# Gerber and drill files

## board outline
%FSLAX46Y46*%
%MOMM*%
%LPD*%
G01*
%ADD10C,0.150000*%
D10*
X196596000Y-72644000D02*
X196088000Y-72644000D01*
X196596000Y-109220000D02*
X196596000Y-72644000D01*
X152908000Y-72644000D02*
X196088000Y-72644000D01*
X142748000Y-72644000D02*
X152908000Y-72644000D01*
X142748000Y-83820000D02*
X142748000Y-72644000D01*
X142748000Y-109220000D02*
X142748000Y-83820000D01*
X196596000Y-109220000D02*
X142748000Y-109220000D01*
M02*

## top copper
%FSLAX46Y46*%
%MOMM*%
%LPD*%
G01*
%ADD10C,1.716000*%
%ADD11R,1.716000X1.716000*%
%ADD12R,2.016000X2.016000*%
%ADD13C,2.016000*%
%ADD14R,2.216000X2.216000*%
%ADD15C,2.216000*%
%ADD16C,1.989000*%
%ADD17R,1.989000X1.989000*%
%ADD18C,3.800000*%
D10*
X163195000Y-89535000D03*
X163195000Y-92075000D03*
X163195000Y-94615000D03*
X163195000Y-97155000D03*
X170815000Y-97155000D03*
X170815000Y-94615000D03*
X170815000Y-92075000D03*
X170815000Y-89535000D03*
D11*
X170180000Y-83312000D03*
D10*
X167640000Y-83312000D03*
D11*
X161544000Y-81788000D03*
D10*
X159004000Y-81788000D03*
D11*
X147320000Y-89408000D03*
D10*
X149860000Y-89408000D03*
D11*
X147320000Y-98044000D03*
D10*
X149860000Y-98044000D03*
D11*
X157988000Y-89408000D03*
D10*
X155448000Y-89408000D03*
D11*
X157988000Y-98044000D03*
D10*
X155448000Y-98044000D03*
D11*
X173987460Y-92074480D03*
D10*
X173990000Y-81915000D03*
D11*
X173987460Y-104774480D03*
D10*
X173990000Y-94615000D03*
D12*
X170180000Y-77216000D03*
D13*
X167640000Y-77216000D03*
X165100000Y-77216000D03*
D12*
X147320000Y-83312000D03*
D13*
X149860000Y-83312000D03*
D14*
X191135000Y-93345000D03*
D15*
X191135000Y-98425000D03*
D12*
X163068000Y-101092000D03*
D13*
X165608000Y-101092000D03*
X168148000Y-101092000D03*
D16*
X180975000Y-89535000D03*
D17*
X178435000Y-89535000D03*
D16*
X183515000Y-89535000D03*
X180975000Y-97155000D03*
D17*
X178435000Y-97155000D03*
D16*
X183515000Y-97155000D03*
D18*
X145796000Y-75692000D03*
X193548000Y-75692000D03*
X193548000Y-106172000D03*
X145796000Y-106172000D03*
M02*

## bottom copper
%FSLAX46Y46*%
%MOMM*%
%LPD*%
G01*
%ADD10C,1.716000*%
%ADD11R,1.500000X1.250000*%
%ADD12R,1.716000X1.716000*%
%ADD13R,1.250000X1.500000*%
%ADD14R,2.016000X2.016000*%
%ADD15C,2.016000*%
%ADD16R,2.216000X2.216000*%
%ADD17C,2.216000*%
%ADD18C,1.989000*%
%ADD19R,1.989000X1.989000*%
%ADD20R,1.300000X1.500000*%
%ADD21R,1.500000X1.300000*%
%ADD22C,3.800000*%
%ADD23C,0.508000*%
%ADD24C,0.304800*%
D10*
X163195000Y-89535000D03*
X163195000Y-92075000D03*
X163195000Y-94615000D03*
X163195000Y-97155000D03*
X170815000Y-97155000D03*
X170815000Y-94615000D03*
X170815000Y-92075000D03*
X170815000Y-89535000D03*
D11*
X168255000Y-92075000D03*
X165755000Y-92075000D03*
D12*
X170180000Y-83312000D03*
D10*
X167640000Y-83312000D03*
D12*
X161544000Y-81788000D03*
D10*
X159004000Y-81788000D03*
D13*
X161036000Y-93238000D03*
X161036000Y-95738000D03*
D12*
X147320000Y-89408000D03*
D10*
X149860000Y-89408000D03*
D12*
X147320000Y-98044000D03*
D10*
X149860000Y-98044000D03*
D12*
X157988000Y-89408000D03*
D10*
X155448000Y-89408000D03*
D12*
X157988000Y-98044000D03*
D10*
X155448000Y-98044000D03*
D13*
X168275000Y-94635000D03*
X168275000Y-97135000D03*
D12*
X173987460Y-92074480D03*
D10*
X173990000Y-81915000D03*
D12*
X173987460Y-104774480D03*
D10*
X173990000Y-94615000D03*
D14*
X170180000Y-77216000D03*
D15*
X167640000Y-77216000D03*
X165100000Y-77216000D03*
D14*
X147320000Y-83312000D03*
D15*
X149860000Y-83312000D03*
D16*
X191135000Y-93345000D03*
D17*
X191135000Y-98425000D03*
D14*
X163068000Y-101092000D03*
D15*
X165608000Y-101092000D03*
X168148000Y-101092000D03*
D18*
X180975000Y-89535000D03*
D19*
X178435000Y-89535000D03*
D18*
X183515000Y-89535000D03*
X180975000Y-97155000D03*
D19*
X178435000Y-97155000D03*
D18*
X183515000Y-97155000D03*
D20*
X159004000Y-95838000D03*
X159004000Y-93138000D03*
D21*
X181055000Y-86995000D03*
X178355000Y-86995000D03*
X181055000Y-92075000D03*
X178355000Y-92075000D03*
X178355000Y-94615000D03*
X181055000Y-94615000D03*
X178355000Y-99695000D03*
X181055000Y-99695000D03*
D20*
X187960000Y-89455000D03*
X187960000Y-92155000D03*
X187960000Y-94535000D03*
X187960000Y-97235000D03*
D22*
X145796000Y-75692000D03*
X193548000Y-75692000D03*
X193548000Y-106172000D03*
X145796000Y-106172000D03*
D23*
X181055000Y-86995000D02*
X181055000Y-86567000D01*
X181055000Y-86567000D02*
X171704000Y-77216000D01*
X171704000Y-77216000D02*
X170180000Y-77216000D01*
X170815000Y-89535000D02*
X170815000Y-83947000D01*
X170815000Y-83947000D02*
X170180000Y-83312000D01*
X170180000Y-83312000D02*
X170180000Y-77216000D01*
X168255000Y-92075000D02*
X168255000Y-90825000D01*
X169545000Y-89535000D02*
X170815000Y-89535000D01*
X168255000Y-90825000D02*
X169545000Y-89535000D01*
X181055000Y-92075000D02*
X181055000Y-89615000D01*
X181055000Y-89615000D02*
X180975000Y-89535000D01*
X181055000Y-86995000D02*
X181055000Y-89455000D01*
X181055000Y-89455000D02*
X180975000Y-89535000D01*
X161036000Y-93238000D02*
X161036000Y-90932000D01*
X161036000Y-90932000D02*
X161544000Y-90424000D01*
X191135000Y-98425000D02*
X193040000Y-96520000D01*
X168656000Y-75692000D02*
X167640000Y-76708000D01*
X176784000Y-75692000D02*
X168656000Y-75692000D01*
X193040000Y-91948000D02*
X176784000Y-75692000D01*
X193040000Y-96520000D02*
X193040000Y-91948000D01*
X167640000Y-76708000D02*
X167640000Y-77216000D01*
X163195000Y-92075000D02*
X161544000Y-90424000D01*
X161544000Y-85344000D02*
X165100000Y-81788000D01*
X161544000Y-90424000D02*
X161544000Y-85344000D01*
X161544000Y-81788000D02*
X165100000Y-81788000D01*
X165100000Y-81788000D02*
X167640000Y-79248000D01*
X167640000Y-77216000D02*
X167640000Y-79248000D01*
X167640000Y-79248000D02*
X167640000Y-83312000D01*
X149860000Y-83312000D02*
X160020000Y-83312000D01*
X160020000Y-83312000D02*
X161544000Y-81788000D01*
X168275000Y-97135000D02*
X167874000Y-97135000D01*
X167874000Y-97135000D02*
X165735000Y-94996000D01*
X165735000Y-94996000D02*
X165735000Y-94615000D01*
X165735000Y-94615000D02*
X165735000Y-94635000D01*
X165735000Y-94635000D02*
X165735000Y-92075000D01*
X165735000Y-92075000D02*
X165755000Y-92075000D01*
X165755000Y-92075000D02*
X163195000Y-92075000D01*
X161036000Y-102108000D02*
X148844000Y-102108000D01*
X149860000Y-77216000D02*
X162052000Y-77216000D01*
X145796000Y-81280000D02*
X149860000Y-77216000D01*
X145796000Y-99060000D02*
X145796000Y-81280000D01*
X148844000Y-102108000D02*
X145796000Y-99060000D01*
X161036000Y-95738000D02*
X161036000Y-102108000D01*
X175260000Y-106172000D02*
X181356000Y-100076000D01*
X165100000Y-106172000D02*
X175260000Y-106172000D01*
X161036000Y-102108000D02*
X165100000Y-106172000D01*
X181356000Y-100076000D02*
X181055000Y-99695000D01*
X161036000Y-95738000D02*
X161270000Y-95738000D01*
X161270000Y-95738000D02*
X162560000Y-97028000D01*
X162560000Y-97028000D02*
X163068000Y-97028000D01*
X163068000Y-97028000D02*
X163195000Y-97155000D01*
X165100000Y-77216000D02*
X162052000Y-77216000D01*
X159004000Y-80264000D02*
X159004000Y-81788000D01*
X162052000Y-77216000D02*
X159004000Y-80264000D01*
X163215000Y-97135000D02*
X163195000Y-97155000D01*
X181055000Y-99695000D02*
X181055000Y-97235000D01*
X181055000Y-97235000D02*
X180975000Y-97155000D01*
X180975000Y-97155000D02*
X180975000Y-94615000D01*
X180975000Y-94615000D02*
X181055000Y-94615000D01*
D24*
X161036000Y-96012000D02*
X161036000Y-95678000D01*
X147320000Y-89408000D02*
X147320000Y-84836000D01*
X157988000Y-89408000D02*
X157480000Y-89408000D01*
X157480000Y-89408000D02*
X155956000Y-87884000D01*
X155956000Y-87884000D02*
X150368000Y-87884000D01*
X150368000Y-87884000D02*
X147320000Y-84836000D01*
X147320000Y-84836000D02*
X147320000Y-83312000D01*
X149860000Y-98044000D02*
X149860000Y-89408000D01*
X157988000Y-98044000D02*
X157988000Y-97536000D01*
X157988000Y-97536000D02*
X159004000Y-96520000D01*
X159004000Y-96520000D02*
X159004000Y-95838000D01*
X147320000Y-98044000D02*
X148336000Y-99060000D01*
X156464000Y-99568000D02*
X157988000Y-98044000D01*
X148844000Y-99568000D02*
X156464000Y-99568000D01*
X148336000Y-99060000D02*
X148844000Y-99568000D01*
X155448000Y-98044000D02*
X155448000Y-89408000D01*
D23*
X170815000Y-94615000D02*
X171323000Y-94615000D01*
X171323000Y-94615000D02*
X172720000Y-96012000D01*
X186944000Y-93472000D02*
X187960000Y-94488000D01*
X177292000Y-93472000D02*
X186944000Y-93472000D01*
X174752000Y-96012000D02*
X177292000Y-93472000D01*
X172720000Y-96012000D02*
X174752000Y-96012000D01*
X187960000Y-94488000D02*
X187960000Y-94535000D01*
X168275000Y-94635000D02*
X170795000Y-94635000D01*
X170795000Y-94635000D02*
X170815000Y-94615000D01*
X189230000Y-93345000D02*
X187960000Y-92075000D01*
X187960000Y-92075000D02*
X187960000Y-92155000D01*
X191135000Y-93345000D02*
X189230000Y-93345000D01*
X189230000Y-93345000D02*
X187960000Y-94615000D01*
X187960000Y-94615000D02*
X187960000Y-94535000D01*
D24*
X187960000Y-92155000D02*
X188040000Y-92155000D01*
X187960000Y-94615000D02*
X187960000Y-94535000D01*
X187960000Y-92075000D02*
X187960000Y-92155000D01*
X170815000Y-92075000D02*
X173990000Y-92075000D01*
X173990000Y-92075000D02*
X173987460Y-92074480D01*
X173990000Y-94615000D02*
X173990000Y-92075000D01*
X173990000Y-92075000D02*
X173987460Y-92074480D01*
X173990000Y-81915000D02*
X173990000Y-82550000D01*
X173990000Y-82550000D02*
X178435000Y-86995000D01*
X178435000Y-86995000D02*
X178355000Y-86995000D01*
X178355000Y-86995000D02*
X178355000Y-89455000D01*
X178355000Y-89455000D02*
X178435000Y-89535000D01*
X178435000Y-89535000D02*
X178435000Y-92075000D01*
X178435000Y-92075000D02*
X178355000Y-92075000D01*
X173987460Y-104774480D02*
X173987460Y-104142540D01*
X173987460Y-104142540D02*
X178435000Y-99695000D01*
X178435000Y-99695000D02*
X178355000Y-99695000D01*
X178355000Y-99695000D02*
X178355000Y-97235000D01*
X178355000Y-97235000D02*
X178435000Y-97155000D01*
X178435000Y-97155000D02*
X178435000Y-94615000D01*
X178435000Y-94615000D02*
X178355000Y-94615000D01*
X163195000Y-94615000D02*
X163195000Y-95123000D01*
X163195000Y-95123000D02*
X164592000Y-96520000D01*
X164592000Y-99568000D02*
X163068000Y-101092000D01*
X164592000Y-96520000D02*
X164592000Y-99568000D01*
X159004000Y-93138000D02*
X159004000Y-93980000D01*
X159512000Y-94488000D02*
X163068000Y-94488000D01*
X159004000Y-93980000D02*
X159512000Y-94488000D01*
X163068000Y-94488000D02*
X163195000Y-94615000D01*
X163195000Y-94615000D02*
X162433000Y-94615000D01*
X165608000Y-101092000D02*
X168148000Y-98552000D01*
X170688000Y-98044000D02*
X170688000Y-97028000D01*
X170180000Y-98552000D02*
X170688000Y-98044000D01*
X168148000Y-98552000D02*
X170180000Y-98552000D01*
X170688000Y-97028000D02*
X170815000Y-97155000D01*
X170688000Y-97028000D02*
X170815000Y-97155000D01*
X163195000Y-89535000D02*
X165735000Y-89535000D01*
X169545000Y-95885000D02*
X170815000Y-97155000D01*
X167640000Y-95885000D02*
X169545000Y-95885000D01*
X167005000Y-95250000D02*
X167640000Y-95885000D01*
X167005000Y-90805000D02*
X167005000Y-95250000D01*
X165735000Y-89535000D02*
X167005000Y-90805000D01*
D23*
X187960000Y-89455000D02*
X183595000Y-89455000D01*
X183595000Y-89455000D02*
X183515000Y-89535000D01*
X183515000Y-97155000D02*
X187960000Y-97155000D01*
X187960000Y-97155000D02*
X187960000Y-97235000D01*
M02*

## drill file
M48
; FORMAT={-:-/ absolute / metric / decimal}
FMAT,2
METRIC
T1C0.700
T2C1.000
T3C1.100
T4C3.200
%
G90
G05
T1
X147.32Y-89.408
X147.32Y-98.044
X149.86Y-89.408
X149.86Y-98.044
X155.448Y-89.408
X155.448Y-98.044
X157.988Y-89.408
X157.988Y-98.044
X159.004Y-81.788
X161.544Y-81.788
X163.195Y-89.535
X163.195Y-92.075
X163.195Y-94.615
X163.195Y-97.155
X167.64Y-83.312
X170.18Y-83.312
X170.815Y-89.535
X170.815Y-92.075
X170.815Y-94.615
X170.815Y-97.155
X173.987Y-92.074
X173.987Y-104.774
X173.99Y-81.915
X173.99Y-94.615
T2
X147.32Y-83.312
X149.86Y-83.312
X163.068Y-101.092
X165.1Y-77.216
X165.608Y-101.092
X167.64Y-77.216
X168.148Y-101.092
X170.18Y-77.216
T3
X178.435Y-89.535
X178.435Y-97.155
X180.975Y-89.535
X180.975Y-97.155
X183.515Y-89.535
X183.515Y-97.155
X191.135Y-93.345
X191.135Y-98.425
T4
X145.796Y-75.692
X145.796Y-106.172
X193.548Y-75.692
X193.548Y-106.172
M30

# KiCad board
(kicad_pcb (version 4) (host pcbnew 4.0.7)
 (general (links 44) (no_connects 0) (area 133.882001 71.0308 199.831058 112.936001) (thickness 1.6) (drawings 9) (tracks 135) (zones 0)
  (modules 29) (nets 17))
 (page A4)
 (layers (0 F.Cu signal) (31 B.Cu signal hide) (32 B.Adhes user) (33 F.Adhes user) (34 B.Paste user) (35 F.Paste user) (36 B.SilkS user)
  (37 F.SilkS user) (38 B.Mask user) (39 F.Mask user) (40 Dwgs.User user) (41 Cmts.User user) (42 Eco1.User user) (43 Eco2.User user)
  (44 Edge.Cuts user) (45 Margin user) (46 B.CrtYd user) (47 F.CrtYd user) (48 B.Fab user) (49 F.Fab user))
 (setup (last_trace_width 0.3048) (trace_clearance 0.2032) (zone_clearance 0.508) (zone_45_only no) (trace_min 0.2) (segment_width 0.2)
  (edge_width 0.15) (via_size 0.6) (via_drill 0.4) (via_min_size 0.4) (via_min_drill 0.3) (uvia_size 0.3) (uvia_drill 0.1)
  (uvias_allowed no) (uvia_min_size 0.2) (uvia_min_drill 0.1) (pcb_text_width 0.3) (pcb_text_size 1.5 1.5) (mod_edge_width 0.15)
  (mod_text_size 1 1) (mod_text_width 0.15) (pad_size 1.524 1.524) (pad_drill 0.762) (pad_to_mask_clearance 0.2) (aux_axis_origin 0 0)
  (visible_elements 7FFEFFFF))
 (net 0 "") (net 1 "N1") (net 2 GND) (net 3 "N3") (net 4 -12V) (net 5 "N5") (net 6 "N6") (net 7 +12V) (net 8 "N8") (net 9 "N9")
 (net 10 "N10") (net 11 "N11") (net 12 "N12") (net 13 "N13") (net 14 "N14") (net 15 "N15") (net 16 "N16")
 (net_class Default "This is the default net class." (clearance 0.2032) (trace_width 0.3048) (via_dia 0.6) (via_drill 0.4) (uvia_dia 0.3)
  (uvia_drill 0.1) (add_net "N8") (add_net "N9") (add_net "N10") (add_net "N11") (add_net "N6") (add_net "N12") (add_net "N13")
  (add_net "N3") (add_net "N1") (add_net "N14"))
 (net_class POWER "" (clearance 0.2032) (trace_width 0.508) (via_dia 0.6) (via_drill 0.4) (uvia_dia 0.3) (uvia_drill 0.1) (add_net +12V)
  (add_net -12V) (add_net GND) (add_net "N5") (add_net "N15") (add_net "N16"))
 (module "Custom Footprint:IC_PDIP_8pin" (layer F.Cu) (at 167.005 93.345 270)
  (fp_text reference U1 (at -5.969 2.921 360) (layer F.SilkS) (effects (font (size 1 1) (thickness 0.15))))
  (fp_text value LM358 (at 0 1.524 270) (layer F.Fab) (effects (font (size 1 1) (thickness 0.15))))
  (pad 1 thru_hole circle (at -3.81 3.81 270) (size 1.716 1.716) (drill 0.7) (layers *.Cu *.Mask F.SilkS) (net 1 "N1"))
  (pad 2 thru_hole circle (at -1.27 3.81 270) (size 1.716 1.716) (drill 0.7) (layers *.Cu *.Mask F.SilkS) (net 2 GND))
  (pad 3 thru_hole circle (at 1.27 3.81 270) (size 1.716 1.716) (drill 0.7) (layers *.Cu *.Mask F.SilkS) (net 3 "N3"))
  (pad 4 thru_hole circle (at 3.81 3.81 270) (size 1.716 1.716) (drill 0.7) (layers *.Cu *.Mask F.SilkS) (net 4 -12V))
  (pad 5 thru_hole circle (at 3.81 -3.81 270) (size 1.716 1.716) (drill 0.7) (layers *.Cu *.Mask F.SilkS) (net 1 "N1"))
  (pad 6 thru_hole circle (at 1.27 -3.81 270) (size 1.716 1.716) (drill 0.7) (layers *.Cu *.Mask F.SilkS) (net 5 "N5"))
  (pad 7 thru_hole circle (at -1.27 -3.81 270) (size 1.716 1.716) (drill 0.7) (layers *.Cu *.Mask F.SilkS) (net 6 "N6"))
  (pad 8 thru_hole circle (at -3.81 -3.81 270) (size 1.716 1.716) (drill 0.7) (layers *.Cu *.Mask F.SilkS) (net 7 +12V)))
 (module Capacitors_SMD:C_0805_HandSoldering (layer B.Cu) (at 167.005 92.075 180)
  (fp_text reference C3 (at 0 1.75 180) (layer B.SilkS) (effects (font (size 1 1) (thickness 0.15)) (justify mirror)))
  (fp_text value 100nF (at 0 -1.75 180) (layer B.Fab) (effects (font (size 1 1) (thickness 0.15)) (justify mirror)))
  (pad 1 smd rect (at -1.25 0 180) (size 1.5 1.25) (layers B.Cu B.Paste B.Mask) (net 7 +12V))
  (pad 2 smd rect (at 1.25 0 180) (size 1.5 1.25) (layers B.Cu B.Paste B.Mask) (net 2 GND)))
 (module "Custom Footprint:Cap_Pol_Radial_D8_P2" (layer F.Cu) (at 170.18 83.312 180)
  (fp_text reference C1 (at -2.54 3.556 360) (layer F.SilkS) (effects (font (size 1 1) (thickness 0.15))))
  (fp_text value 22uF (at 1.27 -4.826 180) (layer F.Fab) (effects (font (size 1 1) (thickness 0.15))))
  (pad 1 thru_hole rect (at 0 0 180) (size 1.716 1.716) (drill 0.7) (layers *.Cu *.Mask F.SilkS) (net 7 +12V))
  (pad 2 thru_hole circle (at 2.54 0 180) (size 1.716 1.716) (drill 0.7) (layers *.Cu *.Mask F.SilkS) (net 2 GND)))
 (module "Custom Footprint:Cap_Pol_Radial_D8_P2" (layer F.Cu) (at 161.544 81.788 180)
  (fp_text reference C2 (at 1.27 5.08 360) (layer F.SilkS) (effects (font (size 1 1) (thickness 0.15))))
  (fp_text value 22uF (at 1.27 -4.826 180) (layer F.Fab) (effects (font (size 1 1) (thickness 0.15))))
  (pad 1 thru_hole rect (at 0 0 180) (size 1.716 1.716) (drill 0.7) (layers *.Cu *.Mask F.SilkS) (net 2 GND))
  (pad 2 thru_hole circle (at 2.54 0 180) (size 1.716 1.716) (drill 0.7) (layers *.Cu *.Mask F.SilkS) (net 4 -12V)))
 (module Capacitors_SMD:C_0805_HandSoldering (layer B.Cu) (at 161.036 94.488 270)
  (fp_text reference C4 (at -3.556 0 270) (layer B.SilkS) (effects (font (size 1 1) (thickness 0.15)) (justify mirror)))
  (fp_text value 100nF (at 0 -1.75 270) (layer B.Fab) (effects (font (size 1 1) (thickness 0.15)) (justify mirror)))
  (pad 1 smd rect (at -1.25 0 270) (size 1.5 1.25) (layers B.Cu B.Paste B.Mask) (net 2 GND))
  (pad 2 smd rect (at 1.25 0 270) (size 1.5 1.25) (layers B.Cu B.Paste B.Mask) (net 4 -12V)))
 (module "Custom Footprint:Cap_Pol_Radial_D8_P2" (layer F.Cu) (at 147.32 89.408)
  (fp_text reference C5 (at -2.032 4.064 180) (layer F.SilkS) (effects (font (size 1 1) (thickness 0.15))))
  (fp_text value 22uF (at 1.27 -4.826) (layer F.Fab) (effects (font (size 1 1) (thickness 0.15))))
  (pad 1 thru_hole rect (at 0 0) (size 1.716 1.716) (drill 0.7) (layers *.Cu *.Mask F.SilkS) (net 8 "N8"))
  (pad 2 thru_hole circle (at 2.54 0) (size 1.716 1.716) (drill 0.7) (layers *.Cu *.Mask F.SilkS) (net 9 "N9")))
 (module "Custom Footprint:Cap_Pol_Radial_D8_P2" (layer F.Cu) (at 147.32 98.044)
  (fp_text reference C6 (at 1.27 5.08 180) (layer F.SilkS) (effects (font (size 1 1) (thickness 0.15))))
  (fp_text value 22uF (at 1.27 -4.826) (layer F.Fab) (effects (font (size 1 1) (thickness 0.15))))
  (pad 1 thru_hole rect (at 0 0) (size 1.716 1.716) (drill 0.7) (layers *.Cu *.Mask F.SilkS) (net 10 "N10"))
  (pad 2 thru_hole circle (at 2.54 0) (size 1.716 1.716) (drill 0.7) (layers *.Cu *.Mask F.SilkS) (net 9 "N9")))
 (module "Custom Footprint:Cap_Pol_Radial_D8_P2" (layer F.Cu) (at 157.988 89.408 180)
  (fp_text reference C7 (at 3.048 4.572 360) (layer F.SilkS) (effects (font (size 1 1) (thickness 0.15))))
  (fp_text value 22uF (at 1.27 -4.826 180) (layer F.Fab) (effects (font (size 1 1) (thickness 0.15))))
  (pad 1 thru_hole rect (at 0 0 180) (size 1.716 1.716) (drill 0.7) (layers *.Cu *.Mask F.SilkS) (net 8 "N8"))
  (pad 2 thru_hole circle (at 2.54 0 180) (size 1.716 1.716) (drill 0.7) (layers *.Cu *.Mask F.SilkS) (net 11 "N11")))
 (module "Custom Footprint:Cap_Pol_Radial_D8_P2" (layer F.Cu) (at 157.988 98.044 180)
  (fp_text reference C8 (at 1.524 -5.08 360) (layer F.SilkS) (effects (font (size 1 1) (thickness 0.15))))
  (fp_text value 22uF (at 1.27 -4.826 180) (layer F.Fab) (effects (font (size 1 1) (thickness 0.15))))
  (pad 1 thru_hole rect (at 0 0 180) (size 1.716 1.716) (drill 0.7) (layers *.Cu *.Mask F.SilkS) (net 10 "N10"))
  (pad 2 thru_hole circle (at 2.54 0 180) (size 1.716 1.716) (drill 0.7) (layers *.Cu *.Mask F.SilkS) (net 11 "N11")))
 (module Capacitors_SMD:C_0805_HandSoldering (layer B.Cu) (at 168.275 95.885 270)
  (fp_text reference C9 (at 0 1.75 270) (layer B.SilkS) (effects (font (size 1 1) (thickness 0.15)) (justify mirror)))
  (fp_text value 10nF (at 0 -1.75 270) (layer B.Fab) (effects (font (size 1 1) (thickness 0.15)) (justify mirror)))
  (pad 1 smd rect (at -1.25 0 270) (size 1.5 1.25) (layers B.Cu B.Paste B.Mask) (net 5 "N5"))
  (pad 2 smd rect (at 1.25 0 270) (size 1.5 1.25) (layers B.Cu B.Paste B.Mask) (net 2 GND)))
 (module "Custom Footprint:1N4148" (layer F.Cu) (at 173.99 92.075 90)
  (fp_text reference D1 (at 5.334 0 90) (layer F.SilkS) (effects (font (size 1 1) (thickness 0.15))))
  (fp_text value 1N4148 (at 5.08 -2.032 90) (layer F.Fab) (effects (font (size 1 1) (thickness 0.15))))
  (pad 1 thru_hole rect (at 0.00052 -0.00254 270) (size 1.716 1.716) (drill 0.7) (layers *.Cu *.Mask F.SilkS) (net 6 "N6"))
  (pad 2 thru_hole circle (at 10.16 0 90) (size 1.716 1.716) (drill 0.7) (layers *.Cu *.Mask F.SilkS) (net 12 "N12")))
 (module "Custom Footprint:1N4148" (layer F.Cu) (at 173.99 104.775 90)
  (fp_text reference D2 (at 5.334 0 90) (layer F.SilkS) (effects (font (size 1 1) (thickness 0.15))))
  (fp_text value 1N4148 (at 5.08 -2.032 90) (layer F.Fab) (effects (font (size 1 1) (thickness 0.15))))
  (pad 1 thru_hole rect (at 0.00052 -0.00254 270) (size 1.716 1.716) (drill 0.7) (layers *.Cu *.Mask F.SilkS) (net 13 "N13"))
  (pad 2 thru_hole circle (at 10.16 0 90) (size 1.716 1.716) (drill 0.7) (layers *.Cu *.Mask F.SilkS) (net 6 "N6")))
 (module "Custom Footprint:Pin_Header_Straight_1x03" (layer F.Cu) (at 170.18 77.216 270)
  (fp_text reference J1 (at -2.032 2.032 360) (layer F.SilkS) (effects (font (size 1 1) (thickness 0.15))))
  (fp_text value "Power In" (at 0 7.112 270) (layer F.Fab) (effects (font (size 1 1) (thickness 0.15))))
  (pad 1 thru_hole rect (at 0 0 270) (size 2.016 2.016) (drill 1) (layers *.Cu *.Mask F.SilkS) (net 7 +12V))
  (pad 2 thru_hole circle (at 0 2.54 270) (size 2.016 2.016) (drill 1) (layers *.Cu *.Mask F.SilkS) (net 2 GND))
  (pad 3 thru_hole circle (at 0 5.08 270) (size 2.016 2.016) (drill 1) (layers *.Cu *.Mask F.SilkS) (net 4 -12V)))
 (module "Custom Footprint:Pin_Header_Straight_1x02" (layer F.Cu) (at 147.32 83.312 90)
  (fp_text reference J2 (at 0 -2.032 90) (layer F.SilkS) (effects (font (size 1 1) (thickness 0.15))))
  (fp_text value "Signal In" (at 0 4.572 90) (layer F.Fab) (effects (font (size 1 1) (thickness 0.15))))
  (pad 1 thru_hole rect (at 0 0 90) (size 2.016 2.016) (drill 1) (layers *.Cu *.Mask F.SilkS) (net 8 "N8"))
  (pad 2 thru_hole circle (at 0 2.54 90) (size 2.016 2.016) (drill 1) (layers *.Cu *.Mask F.SilkS) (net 2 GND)))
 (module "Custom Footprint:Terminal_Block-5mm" (layer F.Cu) (at 191.135 95.885 270)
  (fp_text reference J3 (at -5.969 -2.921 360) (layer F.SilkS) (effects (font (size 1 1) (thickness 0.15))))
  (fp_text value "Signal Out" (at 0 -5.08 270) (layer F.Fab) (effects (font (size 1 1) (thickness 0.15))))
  (pad 1 thru_hole rect (at -2.54 0 270) (size 2.216 2.216) (drill 1.1) (layers *.Cu *.Mask F.SilkS) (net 5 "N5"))
  (pad 2 thru_hole circle (at 2.54 0 270) (size 2.216 2.216) (drill 1.1) (layers *.Cu *.Mask F.SilkS) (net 2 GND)))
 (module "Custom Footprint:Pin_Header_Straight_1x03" (layer F.Cu) (at 163.068 101.092 90)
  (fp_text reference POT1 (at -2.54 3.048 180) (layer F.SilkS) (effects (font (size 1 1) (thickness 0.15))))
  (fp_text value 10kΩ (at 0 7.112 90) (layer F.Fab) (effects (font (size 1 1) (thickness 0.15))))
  (pad 1 thru_hole rect (at 0 0 90) (size 2.016 2.016) (drill 1) (layers *.Cu *.Mask F.SilkS) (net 3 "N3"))
  (pad 2 thru_hole circle (at 0 2.54 90) (size 2.016 2.016) (drill 1) (layers *.Cu *.Mask F.SilkS) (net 1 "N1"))
  (pad 3 thru_hole circle (at 0 5.08 90) (size 2.016 2.016) (drill 1) (layers *.Cu *.Mask F.SilkS) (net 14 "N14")))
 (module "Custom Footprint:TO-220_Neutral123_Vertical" (layer F.Cu) (at 180.975 89.535)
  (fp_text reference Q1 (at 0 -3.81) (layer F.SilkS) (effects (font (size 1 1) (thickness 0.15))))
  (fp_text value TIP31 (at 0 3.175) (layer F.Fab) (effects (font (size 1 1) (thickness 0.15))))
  (pad 2 thru_hole circle (at 0 0 90) (size 1.989 1.989) (drill 1.1) (layers *.Cu *.Mask F.SilkS) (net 7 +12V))
  (pad 1 thru_hole rect (at -2.54 0 90) (size 1.989 1.989) (drill 1.1) (layers *.Cu *.Mask F.SilkS) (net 12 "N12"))
  (pad 3 thru_hole circle (at 2.54 0 90) (size 1.989 1.989) (drill 1.1) (layers *.Cu *.Mask F.SilkS) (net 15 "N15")))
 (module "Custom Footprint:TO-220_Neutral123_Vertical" (layer F.Cu) (at 180.975 97.155)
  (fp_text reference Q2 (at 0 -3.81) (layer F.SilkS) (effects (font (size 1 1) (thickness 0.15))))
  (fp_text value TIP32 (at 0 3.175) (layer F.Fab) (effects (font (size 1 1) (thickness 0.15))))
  (pad 2 thru_hole circle (at 0 0 90) (size 1.989 1.989) (drill 1.1) (layers *.Cu *.Mask F.SilkS) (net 4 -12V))
  (pad 1 thru_hole rect (at -2.54 0 90) (size 1.989 1.989) (drill 1.1) (layers *.Cu *.Mask F.SilkS) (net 13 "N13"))
  (pad 3 thru_hole circle (at 2.54 0 90) (size 1.989 1.989) (drill 1.1) (layers *.Cu *.Mask F.SilkS) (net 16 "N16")))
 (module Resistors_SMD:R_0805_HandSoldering (layer B.Cu) (at 159.004 94.488 90)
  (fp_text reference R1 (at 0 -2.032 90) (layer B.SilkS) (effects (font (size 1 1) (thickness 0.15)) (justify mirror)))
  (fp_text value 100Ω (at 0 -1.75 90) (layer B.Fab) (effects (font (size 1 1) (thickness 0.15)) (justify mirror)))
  (pad 1 smd rect (at -1.35 0 90) (size 1.5 1.3) (layers B.Cu B.Paste B.Mask) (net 10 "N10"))
  (pad 2 smd rect (at 1.35 0 90) (size 1.5 1.3) (layers B.Cu B.Paste B.Mask) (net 3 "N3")))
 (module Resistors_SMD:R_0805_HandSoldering (layer B.Cu) (at 179.705 86.995 180)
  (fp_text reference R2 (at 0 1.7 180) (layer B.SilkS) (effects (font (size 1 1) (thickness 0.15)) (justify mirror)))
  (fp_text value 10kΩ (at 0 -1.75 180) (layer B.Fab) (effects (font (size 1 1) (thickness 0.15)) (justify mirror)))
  (pad 1 smd rect (at -1.35 0 180) (size 1.5 1.3) (layers B.Cu B.Paste B.Mask) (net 7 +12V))
  (pad 2 smd rect (at 1.35 0 180) (size 1.5 1.3) (layers B.Cu B.Paste B.Mask) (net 12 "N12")))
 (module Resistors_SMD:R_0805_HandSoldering (layer B.Cu) (at 179.705 92.075 180)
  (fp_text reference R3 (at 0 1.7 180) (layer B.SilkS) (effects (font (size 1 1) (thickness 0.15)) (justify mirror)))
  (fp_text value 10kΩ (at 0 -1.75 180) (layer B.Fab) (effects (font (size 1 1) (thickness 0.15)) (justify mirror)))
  (pad 1 smd rect (at -1.35 0 180) (size 1.5 1.3) (layers B.Cu B.Paste B.Mask) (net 7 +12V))
  (pad 2 smd rect (at 1.35 0 180) (size 1.5 1.3) (layers B.Cu B.Paste B.Mask) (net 12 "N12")))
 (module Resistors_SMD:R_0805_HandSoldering (layer B.Cu) (at 179.705 94.615)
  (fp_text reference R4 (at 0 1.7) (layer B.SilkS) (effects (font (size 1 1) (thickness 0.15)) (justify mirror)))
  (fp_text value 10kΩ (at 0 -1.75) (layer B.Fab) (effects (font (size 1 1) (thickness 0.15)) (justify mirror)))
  (pad 1 smd rect (at -1.35 0) (size 1.5 1.3) (layers B.Cu B.Paste B.Mask) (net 13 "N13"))
  (pad 2 smd rect (at 1.35 0) (size 1.5 1.3) (layers B.Cu B.Paste B.Mask) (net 4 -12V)))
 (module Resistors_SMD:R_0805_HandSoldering (layer B.Cu) (at 179.705 99.695)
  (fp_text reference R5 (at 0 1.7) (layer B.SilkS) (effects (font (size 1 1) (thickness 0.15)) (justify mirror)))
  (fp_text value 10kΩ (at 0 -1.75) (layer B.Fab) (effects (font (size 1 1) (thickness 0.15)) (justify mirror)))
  (pad 1 smd rect (at -1.35 0) (size 1.5 1.3) (layers B.Cu B.Paste B.Mask) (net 13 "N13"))
  (pad 2 smd rect (at 1.35 0) (size 1.5 1.3) (layers B.Cu B.Paste B.Mask) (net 4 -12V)))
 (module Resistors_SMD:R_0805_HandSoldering (layer B.Cu) (at 187.96 90.805 270)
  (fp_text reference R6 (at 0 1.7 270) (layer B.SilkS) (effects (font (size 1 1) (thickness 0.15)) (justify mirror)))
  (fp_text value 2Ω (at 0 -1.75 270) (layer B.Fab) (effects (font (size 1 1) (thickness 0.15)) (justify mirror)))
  (pad 1 smd rect (at -1.35 0 270) (size 1.5 1.3) (layers B.Cu B.Paste B.Mask) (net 15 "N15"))
  (pad 2 smd rect (at 1.35 0 270) (size 1.5 1.3) (layers B.Cu B.Paste B.Mask) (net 5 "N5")))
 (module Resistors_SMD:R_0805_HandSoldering (layer B.Cu) (at 187.96 95.885 270)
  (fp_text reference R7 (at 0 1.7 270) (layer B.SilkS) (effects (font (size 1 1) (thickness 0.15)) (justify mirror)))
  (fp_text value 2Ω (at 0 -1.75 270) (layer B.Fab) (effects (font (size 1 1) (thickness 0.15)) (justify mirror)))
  (pad 1 smd rect (at -1.35 0 270) (size 1.5 1.3) (layers B.Cu B.Paste B.Mask) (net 5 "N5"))
  (pad 2 smd rect (at 1.35 0 270) (size 1.5 1.3) (layers B.Cu B.Paste B.Mask) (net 16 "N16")))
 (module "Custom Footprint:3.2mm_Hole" (layer F.Cu) (at 145.796 75.692)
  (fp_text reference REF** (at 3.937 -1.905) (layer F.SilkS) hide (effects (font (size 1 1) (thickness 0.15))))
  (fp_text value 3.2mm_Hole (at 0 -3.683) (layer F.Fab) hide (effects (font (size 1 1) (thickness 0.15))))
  (pad 1 thru_hole circle (at 0 0) (size 3.8 3.8) (drill 3.2) (layers *.Cu *.Mask F.SilkS)))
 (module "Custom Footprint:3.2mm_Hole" (layer F.Cu) (at 193.548 75.692)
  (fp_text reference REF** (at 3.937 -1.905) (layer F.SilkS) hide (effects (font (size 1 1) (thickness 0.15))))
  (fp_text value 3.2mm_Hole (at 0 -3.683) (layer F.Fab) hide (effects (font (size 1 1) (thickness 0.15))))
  (pad 1 thru_hole circle (at 0 0) (size 3.8 3.8) (drill 3.2) (layers *.Cu *.Mask F.SilkS)))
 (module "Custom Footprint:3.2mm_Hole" (layer F.Cu) (at 193.548 106.172)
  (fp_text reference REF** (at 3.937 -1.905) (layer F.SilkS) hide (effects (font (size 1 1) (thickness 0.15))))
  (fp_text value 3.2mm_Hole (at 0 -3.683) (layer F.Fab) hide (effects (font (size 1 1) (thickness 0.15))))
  (pad 1 thru_hole circle (at 0 0) (size 3.8 3.8) (drill 3.2) (layers *.Cu *.Mask F.SilkS)))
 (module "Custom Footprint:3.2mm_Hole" (layer F.Cu) (at 145.796 106.172)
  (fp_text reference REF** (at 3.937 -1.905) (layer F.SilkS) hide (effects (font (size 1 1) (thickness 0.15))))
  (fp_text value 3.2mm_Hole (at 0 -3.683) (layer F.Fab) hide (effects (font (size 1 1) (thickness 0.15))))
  (pad 1 thru_hole circle (at 0 0) (size 3.8 3.8) (drill 3.2) (layers *.Cu *.Mask F.SilkS)))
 (gr_line (start 196.596 72.644) (end 196.088 72.644) (angle 90) (layer Edge.Cuts) (width 0.15))
 (gr_line (start 196.596 109.22) (end 196.596 72.644) (angle 90) (layer Edge.Cuts) (width 0.15))
 (gr_line (start 152.908 72.644) (end 196.088 72.644) (angle 90) (layer Edge.Cuts) (width 0.15))
 (gr_line (start 142.748 72.644) (end 152.908 72.644) (angle 90) (layer Edge.Cuts) (width 0.15))
 (gr_line (start 142.748 83.82) (end 142.748 72.644) (angle 90) (layer Edge.Cuts) (width 0.15))
 (gr_line (start 142.748 109.22) (end 142.748 83.82) (angle 90) (layer Edge.Cuts) (width 0.15))
 (gr_line (start 196.596 109.22) (end 142.748 109.22) (angle 90) (layer Edge.Cuts) (width 0.15))
 (segment (start 181.055 86.995) (end 181.055 86.567) (width 0.508) (layer B.Cu) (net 7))
 (segment (start 181.055 86.567) (end 171.704 77.216) (width 0.508) (layer B.Cu) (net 7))
 (segment (start 171.704 77.216) (end 170.18 77.216) (width 0.508) (layer B.Cu) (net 7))
 (segment (start 170.815 89.535) (end 170.815 83.947) (width 0.508) (layer B.Cu) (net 7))
 (segment (start 170.815 83.947) (end 170.18 83.312) (width 0.508) (layer B.Cu) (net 7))
 (segment (start 170.18 83.312) (end 170.18 77.216) (width 0.508) (layer B.Cu) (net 7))
 (segment (start 168.255 92.075) (end 168.255 90.825) (width 0.508) (layer B.Cu) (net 7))
 (segment (start 169.545 89.535) (end 170.815 89.535) (width 0.508) (layer B.Cu) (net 7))
 (segment (start 168.255 90.825) (end 169.545 89.535) (width 0.508) (layer B.Cu) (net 7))
 (segment (start 181.055 92.075) (end 181.055 89.615) (width 0.508) (layer B.Cu) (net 7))
 (segment (start 181.055 89.615) (end 180.975 89.535) (width 0.508) (layer B.Cu) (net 7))
 (segment (start 181.055 86.995) (end 181.055 89.455) (width 0.508) (layer B.Cu) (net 7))
 (segment (start 181.055 89.455) (end 180.975 89.535) (width 0.508) (layer B.Cu) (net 7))
 (segment (start 161.036 93.238) (end 161.036 90.932) (width 0.508) (layer B.Cu) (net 2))
 (segment (start 161.036 90.932) (end 161.544 90.424) (width 0.508) (layer B.Cu) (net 2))
 (segment (start 191.135 98.425) (end 193.04 96.52) (width 0.508) (layer B.Cu) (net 2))
 (segment (start 168.656 75.692) (end 167.64 76.708) (width 0.508) (layer B.Cu) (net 2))
 (segment (start 176.784 75.692) (end 168.656 75.692) (width 0.508) (layer B.Cu) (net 2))
 (segment (start 193.04 91.948) (end 176.784 75.692) (width 0.508) (layer B.Cu) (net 2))
 (segment (start 193.04 96.52) (end 193.04 91.948) (width 0.508) (layer B.Cu) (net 2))
 (segment (start 167.64 76.708) (end 167.64 77.216) (width 0.508) (layer B.Cu) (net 2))
 (segment (start 163.195 92.075) (end 161.544 90.424) (width 0.508) (layer B.Cu) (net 2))
 (segment (start 161.544 85.344) (end 165.1 81.788) (width 0.508) (layer B.Cu) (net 2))
 (segment (start 161.544 90.424) (end 161.544 85.344) (width 0.508) (layer B.Cu) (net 2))
 (segment (start 161.544 81.788) (end 165.1 81.788) (width 0.508) (layer B.Cu) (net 2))
 (segment (start 165.1 81.788) (end 167.64 79.248) (width 0.508) (layer B.Cu) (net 2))
 (segment (start 167.64 77.216) (end 167.64 79.248) (width 0.508) (layer B.Cu) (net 2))
 (segment (start 167.64 79.248) (end 167.64 83.312) (width 0.508) (layer B.Cu) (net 2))
 (segment (start 149.86 83.312) (end 160.02 83.312) (width 0.508) (layer B.Cu) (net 2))
 (segment (start 160.02 83.312) (end 161.544 81.788) (width 0.508) (layer B.Cu) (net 2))
 (segment (start 168.275 97.135) (end 167.874 97.135) (width 0.508) (layer B.Cu) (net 2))
 (segment (start 167.874 97.135) (end 165.735 94.996) (width 0.508) (layer B.Cu) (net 2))
 (segment (start 165.735 94.996) (end 165.735 94.615) (width 0.508) (layer B.Cu) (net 2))
 (segment (start 165.735 94.615) (end 165.735 94.635) (width 0.508) (layer B.Cu) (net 2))
 (segment (start 165.735 94.635) (end 165.735 92.075) (width 0.508) (layer B.Cu) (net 2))
 (segment (start 165.735 92.075) (end 165.755 92.075) (width 0.508) (layer B.Cu) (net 2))
 (segment (start 165.755 92.075) (end 163.195 92.075) (width 0.508) (layer B.Cu) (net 2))
 (segment (start 161.036 102.108) (end 148.844 102.108) (width 0.508) (layer B.Cu) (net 4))
 (segment (start 149.86 77.216) (end 162.052 77.216) (width 0.508) (layer B.Cu) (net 4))
 (segment (start 145.796 81.28) (end 149.86 77.216) (width 0.508) (layer B.Cu) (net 4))
 (segment (start 145.796 99.06) (end 145.796 81.28) (width 0.508) (layer B.Cu) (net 4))
 (segment (start 148.844 102.108) (end 145.796 99.06) (width 0.508) (layer B.Cu) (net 4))
 (segment (start 161.036 95.738) (end 161.036 102.108) (width 0.508) (layer B.Cu) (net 4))
 (segment (start 175.26 106.172) (end 181.356 100.076) (width 0.508) (layer B.Cu) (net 4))
 (segment (start 165.1 106.172) (end 175.26 106.172) (width 0.508) (layer B.Cu) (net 4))
 (segment (start 161.036 102.108) (end 165.1 106.172) (width 0.508) (layer B.Cu) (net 4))
 (segment (start 181.356 100.076) (end 181.055 99.695) (width 0.508) (layer B.Cu) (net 4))
 (segment (start 161.036 95.738) (end 161.27 95.738) (width 0.508) (layer B.Cu) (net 4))
 (segment (start 161.27 95.738) (end 162.56 97.028) (width 0.508) (layer B.Cu) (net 4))
 (segment (start 162.56 97.028) (end 163.068 97.028) (width 0.508) (layer B.Cu) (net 4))
 (segment (start 163.068 97.028) (end 163.195 97.155) (width 0.508) (layer B.Cu) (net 4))
 (segment (start 165.1 77.216) (end 162.052 77.216) (width 0.508) (layer B.Cu) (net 4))
 (segment (start 159.004 80.264) (end 159.004 81.788) (width 0.508) (layer B.Cu) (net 4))
 (segment (start 162.052 77.216) (end 159.004 80.264) (width 0.508) (layer B.Cu) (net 4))
 (segment (start 163.215 97.135) (end 163.195 97.155) (width 0.508) (layer B.Cu) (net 4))
 (segment (start 181.055 99.695) (end 181.055 97.235) (width 0.508) (layer B.Cu) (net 4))
 (segment (start 181.055 97.235) (end 180.975 97.155) (width 0.508) (layer B.Cu) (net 4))
 (segment (start 180.975 97.155) (end 180.975 94.615) (width 0.508) (layer B.Cu) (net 4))
 (segment (start 180.975 94.615) (end 181.055 94.615) (width 0.508) (layer B.Cu) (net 4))
 (segment (start 161.036 96.012) (end 161.036 95.678) (width 0.3048) (layer B.Cu) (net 4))
 (segment (start 147.32 89.408) (end 147.32 84.836) (width 0.3048) (layer B.Cu) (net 8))
 (segment (start 157.988 89.408) (end 157.48 89.408) (width 0.3048) (layer B.Cu) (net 8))
 (segment (start 157.48 89.408) (end 155.956 87.884) (width 0.3048) (layer B.Cu) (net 8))
 (segment (start 155.956 87.884) (end 150.368 87.884) (width 0.3048) (layer B.Cu) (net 8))
 (segment (start 150.368 87.884) (end 147.32 84.836) (width 0.3048) (layer B.Cu) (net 8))
 (segment (start 147.32 84.836) (end 147.32 83.312) (width 0.3048) (layer B.Cu) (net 8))
 (segment (start 149.86 98.044) (end 149.86 89.408) (width 0.3048) (layer B.Cu) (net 9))
 (segment (start 157.988 98.044) (end 157.988 97.536) (width 0.3048) (layer B.Cu) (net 10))
 (segment (start 157.988 97.536) (end 159.004 96.52) (width 0.3048) (layer B.Cu) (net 10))
 (segment (start 159.004 96.52) (end 159.004 95.838) (width 0.3048) (layer B.Cu) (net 10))
 (segment (start 147.32 98.044) (end 148.336 99.06) (width 0.3048) (layer B.Cu) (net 10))
 (segment (start 156.464 99.568) (end 157.988 98.044) (width 0.3048) (layer B.Cu) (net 10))
 (segment (start 148.844 99.568) (end 156.464 99.568) (width 0.3048) (layer B.Cu) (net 10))
 (segment (start 148.336 99.06) (end 148.844 99.568) (width 0.3048) (layer B.Cu) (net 10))
 (segment (start 155.448 98.044) (end 155.448 89.408) (width 0.3048) (layer B.Cu) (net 11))
 (segment (start 170.815 94.615) (end 171.323 94.615) (width 0.508) (layer B.Cu) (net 5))
 (segment (start 171.323 94.615) (end 172.72 96.012) (width 0.508) (layer B.Cu) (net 5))
 (segment (start 186.944 93.472) (end 187.96 94.488) (width 0.508) (layer B.Cu) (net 5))
 (segment (start 177.292 93.472) (end 186.944 93.472) (width 0.508) (layer B.Cu) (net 5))
 (segment (start 174.752 96.012) (end 177.292 93.472) (width 0.508) (layer B.Cu) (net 5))
 (segment (start 172.72 96.012) (end 174.752 96.012) (width 0.508) (layer B.Cu) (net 5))
 (segment (start 187.96 94.488) (end 187.96 94.535) (width 0.508) (layer B.Cu) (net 5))
 (segment (start 168.275 94.635) (end 170.795 94.635) (width 0.508) (layer B.Cu) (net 5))
 (segment (start 170.795 94.635) (end 170.815 94.615) (width 0.508) (layer B.Cu) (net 5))
 (segment (start 189.23 93.345) (end 187.96 92.075) (width 0.508) (layer B.Cu) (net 5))
 (segment (start 187.96 92.075) (end 187.96 92.155) (width 0.508) (layer B.Cu) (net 5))
 (segment (start 191.135 93.345) (end 189.23 93.345) (width 0.508) (layer B.Cu) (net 5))
 (segment (start 189.23 93.345) (end 187.96 94.615) (width 0.508) (layer B.Cu) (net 5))
 (segment (start 187.96 94.615) (end 187.96 94.535) (width 0.508) (layer B.Cu) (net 5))
 (segment (start 187.96 92.155) (end 188.04 92.155) (width 0.3048) (layer B.Cu) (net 5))
 (segment (start 187.96 94.615) (end 187.96 94.535) (width 0.3048) (layer B.Cu) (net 5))
 (segment (start 187.96 92.075) (end 187.96 92.155) (width 0.3048) (layer B.Cu) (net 5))
 (segment (start 170.815 92.075) (end 173.99 92.075) (width 0.3048) (layer B.Cu) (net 6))
 (segment (start 173.99 92.075) (end 173.98746 92.07448) (width 0.3048) (layer B.Cu) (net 6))
 (segment (start 173.99 94.615) (end 173.99 92.075) (width 0.3048) (layer B.Cu) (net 6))
 (segment (start 173.99 92.075) (end 173.98746 92.07448) (width 0.3048) (layer B.Cu) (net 6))
 (segment (start 173.99 81.915) (end 173.99 82.55) (width 0.3048) (layer B.Cu) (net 12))
 (segment (start 173.99 82.55) (end 178.435 86.995) (width 0.3048) (layer B.Cu) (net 12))
 (segment (start 178.435 86.995) (end 178.355 86.995) (width 0.3048) (layer B.Cu) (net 12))
 (segment (start 178.355 86.995) (end 178.355 89.455) (width 0.3048) (layer B.Cu) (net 12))
 (segment (start 178.355 89.455) (end 178.435 89.535) (width 0.3048) (layer B.Cu) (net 12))
 (segment (start 178.435 89.535) (end 178.435 92.075) (width 0.3048) (layer B.Cu) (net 12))
 (segment (start 178.435 92.075) (end 178.355 92.075) (width 0.3048) (layer B.Cu) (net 12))
 (segment (start 173.98746 104.77448) (end 173.98746 104.14254) (width 0.3048) (layer B.Cu) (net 13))
 (segment (start 173.98746 104.14254) (end 178.435 99.695) (width 0.3048) (layer B.Cu) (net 13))
 (segment (start 178.435 99.695) (end 178.355 99.695) (width 0.3048) (layer B.Cu) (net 13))
 (segment (start 178.355 99.695) (end 178.355 97.235) (width 0.3048) (layer B.Cu) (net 13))
 (segment (start 178.355 97.235) (end 178.435 97.155) (width 0.3048) (layer B.Cu) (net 13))
 (segment (start 178.435 97.155) (end 178.435 94.615) (width 0.3048) (layer B.Cu) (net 13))
 (segment (start 178.435 94.615) (end 178.355 94.615) (width 0.3048) (layer B.Cu) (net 13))
 (segment (start 163.195 94.615) (end 163.195 95.123) (width 0.3048) (layer B.Cu) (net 3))
 (segment (start 163.195 95.123) (end 164.592 96.52) (width 0.3048) (layer B.Cu) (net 3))
 (segment (start 164.592 99.568) (end 163.068 101.092) (width 0.3048) (layer B.Cu) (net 3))
 (segment (start 164.592 96.52) (end 164.592 99.568) (width 0.3048) (layer B.Cu) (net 3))
 (segment (start 159.004 93.138) (end 159.004 93.98) (width 0.3048) (layer B.Cu) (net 3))
 (segment (start 159.512 94.488) (end 163.068 94.488) (width 0.3048) (layer B.Cu) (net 3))
 (segment (start 159.004 93.98) (end 159.512 94.488) (width 0.3048) (layer B.Cu) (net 3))
 (segment (start 163.068 94.488) (end 163.195 94.615) (width 0.3048) (layer B.Cu) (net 3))
 (segment (start 163.195 94.615) (end 162.433 94.615) (width 0.3048) (layer B.Cu) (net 3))
 (segment (start 165.608 101.092) (end 168.148 98.552) (width 0.3048) (layer B.Cu) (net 1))
 (segment (start 170.688 98.044) (end 170.688 97.028) (width 0.3048) (layer B.Cu) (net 1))
 (segment (start 170.18 98.552) (end 170.688 98.044) (width 0.3048) (layer B.Cu) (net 1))
 (segment (start 168.148 98.552) (end 170.18 98.552) (width 0.3048) (layer B.Cu) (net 1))
 (segment (start 170.688 97.028) (end 170.815 97.155) (width 0.3048) (layer B.Cu) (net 1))
 (segment (start 170.688 97.028) (end 170.815 97.155) (width 0.3048) (layer B.Cu) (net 1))
 (segment (start 163.195 89.535) (end 165.735 89.535) (width 0.3048) (layer B.Cu) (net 1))
 (segment (start 169.545 95.885) (end 170.815 97.155) (width 0.3048) (layer B.Cu) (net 1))
 (segment (start 167.64 95.885) (end 169.545 95.885) (width 0.3048) (layer B.Cu) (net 1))
 (segment (start 167.005 95.25) (end 167.64 95.885) (width 0.3048) (layer B.Cu) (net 1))
 (segment (start 167.005 90.805) (end 167.005 95.25) (width 0.3048) (layer B.Cu) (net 1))
 (segment (start 165.735 89.535) (end 167.005 90.805) (width 0.3048) (layer B.Cu) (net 1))
 (segment (start 187.96 89.455) (end 183.595 89.455) (width 0.508) (layer B.Cu) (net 15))
 (segment (start 183.595 89.455) (end 183.515 89.535) (width 0.508) (layer B.Cu) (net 15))
 (segment (start 183.515 97.155) (end 187.96 97.155) (width 0.508) (layer B.Cu) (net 16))
 (segment (start 187.96 97.155) (end 187.96 97.235) (width 0.508) (layer B.Cu) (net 16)))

